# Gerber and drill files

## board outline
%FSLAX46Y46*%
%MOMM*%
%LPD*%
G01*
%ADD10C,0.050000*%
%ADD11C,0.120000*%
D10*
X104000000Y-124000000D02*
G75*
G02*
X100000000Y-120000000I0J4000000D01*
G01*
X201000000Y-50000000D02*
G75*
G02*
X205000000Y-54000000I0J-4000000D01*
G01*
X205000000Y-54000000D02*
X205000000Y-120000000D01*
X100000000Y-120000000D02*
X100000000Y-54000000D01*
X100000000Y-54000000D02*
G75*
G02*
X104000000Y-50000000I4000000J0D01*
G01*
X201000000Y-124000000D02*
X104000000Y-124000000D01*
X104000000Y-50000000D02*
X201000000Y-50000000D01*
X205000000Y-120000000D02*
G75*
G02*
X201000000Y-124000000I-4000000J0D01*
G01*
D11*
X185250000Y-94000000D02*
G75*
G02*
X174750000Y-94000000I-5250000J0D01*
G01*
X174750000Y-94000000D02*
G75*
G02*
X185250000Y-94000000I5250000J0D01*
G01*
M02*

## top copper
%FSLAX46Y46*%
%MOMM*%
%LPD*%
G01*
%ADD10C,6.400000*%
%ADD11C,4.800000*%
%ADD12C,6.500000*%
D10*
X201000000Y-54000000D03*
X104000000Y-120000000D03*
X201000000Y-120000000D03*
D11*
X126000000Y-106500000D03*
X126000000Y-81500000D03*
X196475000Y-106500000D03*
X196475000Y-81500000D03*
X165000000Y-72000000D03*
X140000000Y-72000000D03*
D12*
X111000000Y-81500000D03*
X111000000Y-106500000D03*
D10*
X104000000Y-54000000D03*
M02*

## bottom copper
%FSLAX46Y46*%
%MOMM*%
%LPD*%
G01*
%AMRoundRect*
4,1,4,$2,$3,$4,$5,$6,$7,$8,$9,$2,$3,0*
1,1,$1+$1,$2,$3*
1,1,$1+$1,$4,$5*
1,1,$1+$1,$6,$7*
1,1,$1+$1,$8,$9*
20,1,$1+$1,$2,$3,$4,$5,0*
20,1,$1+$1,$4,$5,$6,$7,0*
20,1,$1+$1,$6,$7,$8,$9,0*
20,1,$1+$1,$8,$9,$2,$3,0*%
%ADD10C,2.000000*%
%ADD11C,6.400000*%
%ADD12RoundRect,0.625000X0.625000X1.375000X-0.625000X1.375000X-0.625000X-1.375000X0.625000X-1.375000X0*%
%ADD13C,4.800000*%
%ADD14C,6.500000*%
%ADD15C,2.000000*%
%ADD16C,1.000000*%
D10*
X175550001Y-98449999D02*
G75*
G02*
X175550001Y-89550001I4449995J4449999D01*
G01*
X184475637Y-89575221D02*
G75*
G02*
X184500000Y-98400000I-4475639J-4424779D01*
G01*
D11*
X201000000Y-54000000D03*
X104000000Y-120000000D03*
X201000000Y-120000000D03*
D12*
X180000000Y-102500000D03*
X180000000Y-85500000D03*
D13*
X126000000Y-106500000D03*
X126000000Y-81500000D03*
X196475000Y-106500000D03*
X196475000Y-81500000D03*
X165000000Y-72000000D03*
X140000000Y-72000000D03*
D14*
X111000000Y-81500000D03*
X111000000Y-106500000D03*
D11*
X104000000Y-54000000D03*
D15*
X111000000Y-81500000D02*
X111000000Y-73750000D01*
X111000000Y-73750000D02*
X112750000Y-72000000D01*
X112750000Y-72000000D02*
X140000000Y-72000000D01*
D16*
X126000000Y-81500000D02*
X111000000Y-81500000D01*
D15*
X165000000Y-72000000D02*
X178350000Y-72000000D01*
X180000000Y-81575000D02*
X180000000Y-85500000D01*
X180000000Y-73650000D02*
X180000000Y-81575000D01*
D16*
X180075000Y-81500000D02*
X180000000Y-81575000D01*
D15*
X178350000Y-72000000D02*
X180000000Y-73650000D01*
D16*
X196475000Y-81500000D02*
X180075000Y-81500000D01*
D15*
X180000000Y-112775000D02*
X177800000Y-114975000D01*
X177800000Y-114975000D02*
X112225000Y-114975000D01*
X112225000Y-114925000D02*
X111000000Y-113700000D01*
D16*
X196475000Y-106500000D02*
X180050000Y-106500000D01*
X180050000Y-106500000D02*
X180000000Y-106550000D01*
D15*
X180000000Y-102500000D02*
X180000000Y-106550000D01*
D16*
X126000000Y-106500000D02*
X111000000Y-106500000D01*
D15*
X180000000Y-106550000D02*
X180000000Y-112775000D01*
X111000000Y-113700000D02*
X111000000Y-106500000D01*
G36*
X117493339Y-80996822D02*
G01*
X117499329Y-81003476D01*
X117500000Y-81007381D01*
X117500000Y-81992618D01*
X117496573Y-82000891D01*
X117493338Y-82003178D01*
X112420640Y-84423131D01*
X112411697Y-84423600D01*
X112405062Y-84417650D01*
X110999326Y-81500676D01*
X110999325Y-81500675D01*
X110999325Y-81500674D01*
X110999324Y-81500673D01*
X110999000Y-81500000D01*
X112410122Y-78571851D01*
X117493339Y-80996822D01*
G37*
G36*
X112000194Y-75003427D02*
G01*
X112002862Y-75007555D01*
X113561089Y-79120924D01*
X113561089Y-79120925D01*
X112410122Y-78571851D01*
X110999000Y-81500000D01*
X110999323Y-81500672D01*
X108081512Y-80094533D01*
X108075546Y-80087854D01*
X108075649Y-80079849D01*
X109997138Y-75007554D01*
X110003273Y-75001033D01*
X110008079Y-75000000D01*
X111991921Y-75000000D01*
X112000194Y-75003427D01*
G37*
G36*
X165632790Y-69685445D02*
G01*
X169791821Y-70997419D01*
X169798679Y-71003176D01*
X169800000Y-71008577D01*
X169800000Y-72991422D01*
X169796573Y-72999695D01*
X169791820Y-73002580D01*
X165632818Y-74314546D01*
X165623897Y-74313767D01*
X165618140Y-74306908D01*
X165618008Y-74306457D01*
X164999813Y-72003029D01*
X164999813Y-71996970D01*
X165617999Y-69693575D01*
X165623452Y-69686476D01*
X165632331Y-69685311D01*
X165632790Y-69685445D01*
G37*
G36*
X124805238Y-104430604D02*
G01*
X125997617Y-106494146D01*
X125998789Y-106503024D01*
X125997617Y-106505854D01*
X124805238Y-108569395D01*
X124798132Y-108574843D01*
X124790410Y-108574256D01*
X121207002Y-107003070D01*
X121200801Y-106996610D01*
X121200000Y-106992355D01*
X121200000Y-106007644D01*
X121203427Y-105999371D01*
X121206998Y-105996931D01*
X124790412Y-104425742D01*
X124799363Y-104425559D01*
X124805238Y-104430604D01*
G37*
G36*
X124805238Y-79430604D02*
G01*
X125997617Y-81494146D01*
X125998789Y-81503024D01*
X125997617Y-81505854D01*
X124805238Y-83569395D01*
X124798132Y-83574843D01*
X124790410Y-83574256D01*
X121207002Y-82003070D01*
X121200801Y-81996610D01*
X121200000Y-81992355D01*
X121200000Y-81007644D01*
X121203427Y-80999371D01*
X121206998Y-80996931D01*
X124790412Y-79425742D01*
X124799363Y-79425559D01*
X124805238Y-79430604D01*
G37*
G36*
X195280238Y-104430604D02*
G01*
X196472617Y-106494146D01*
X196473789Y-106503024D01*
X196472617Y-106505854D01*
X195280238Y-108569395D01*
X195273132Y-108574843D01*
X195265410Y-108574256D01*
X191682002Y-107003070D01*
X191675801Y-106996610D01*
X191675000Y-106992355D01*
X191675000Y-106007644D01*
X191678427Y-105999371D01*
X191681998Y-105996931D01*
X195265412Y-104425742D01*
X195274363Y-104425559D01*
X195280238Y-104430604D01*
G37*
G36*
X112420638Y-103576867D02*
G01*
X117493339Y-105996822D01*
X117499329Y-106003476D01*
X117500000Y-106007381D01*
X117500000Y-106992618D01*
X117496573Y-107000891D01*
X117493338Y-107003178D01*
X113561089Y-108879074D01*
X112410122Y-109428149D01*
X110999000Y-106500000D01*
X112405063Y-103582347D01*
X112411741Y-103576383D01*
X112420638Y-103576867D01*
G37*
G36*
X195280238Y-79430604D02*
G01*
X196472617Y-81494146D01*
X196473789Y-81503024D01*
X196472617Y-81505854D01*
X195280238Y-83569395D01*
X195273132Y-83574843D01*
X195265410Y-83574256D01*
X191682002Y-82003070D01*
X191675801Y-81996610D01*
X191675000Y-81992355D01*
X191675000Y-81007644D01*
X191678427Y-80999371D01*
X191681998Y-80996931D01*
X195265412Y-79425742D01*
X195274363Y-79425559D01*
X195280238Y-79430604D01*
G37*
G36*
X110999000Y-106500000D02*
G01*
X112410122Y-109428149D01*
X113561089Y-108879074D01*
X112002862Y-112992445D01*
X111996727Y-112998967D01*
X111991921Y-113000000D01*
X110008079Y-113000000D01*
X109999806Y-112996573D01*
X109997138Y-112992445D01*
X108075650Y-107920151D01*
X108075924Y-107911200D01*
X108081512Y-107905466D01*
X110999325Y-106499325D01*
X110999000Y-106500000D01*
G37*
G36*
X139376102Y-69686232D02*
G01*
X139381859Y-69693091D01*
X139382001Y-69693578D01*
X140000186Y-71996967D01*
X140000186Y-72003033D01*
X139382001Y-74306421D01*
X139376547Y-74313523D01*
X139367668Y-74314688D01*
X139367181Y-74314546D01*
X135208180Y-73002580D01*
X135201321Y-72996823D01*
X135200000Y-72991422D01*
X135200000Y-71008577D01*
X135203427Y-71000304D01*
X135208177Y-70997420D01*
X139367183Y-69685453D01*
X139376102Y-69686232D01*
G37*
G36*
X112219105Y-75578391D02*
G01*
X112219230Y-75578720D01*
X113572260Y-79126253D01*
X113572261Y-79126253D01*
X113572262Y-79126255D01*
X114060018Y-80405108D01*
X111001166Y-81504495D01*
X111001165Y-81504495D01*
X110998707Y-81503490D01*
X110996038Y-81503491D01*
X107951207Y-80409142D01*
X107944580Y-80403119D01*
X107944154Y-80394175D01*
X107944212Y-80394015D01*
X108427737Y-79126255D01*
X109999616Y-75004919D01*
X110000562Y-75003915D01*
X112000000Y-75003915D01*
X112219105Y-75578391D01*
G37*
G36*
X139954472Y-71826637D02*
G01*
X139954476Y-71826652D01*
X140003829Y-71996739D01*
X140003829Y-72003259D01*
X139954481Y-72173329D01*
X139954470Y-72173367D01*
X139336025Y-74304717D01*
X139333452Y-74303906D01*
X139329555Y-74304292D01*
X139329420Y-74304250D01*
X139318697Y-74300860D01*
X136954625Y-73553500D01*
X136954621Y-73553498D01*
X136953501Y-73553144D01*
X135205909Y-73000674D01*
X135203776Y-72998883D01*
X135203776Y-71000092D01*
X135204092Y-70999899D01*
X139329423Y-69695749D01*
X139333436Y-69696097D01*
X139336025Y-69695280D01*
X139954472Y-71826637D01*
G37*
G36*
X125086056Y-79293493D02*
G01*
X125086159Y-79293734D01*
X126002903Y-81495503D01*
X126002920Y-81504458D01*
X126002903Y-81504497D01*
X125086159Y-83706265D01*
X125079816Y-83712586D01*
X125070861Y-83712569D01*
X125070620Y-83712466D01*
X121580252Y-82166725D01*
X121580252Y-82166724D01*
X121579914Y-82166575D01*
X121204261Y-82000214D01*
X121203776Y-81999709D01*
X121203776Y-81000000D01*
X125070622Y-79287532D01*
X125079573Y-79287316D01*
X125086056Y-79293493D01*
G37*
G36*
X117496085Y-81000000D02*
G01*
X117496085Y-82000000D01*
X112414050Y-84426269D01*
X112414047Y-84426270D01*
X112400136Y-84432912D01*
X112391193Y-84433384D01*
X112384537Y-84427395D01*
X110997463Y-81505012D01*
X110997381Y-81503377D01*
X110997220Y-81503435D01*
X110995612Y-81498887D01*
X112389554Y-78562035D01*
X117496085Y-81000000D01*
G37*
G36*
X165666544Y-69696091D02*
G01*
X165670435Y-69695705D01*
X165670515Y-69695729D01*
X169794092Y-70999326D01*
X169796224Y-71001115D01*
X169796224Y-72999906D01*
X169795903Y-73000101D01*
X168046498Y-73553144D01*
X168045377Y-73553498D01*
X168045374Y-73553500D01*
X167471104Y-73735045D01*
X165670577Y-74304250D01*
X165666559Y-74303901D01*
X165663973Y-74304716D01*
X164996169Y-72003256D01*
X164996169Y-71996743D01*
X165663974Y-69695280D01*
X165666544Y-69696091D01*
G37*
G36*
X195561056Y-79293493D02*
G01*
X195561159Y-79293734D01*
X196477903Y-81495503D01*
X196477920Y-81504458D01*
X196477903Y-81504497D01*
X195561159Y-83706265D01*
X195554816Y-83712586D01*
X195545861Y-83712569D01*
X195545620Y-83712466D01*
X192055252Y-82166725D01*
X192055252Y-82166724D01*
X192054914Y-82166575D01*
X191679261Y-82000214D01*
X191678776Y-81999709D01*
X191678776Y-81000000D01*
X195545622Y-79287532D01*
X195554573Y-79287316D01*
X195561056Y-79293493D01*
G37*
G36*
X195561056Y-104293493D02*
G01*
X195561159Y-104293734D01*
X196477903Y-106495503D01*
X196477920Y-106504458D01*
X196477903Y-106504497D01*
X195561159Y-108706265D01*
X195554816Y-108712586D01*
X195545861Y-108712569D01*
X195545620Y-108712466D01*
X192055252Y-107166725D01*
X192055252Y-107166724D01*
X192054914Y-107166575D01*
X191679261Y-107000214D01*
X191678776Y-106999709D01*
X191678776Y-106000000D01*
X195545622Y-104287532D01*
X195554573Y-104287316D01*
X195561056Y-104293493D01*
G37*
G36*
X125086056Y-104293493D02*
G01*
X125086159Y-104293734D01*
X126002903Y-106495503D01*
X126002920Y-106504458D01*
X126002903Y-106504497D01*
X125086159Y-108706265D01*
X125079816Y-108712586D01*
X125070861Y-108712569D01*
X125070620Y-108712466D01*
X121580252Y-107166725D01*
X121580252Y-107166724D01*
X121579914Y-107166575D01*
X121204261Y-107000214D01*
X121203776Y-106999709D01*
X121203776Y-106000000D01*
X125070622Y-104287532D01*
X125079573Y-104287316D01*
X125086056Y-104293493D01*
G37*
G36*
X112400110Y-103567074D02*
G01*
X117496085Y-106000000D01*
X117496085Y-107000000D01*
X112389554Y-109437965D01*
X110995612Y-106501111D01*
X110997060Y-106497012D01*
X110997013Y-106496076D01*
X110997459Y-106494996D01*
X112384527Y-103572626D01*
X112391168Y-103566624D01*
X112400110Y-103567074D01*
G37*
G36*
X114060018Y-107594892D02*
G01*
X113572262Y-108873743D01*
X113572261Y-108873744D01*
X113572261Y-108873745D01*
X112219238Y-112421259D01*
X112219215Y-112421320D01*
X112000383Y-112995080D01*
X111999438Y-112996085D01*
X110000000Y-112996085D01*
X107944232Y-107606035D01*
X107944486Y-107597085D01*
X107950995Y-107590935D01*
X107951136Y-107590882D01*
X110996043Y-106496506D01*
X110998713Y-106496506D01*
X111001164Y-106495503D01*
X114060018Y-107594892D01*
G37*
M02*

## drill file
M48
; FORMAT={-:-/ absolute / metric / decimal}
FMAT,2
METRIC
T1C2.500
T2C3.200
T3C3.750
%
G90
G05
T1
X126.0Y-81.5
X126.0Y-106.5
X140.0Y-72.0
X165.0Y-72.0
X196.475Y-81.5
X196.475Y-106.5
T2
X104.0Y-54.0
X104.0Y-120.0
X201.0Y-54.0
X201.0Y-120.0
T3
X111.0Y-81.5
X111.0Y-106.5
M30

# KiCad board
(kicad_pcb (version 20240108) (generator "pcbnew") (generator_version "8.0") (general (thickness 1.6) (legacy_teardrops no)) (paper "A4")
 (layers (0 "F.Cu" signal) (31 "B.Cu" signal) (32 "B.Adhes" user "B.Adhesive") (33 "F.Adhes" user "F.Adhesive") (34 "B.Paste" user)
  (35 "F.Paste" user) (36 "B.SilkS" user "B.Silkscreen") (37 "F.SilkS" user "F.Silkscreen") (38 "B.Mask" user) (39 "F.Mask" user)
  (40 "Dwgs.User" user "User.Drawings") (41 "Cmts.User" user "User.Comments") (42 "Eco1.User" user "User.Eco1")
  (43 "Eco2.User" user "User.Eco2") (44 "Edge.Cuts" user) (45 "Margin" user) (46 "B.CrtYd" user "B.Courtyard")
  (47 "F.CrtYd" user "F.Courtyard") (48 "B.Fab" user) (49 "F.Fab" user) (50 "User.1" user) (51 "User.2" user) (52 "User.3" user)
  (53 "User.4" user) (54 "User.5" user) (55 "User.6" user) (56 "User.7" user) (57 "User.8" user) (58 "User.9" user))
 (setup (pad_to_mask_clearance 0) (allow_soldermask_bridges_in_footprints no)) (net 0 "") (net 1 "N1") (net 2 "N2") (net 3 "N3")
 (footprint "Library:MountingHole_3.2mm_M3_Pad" (layer "F.Cu") (at 201 54)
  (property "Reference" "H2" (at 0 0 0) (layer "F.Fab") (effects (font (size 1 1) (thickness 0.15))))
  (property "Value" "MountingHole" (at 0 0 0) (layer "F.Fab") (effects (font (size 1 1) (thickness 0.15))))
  (pad "1" thru_hole circle (at 0 0) (size 6.4 6.4) (drill 3.2) (layers "*.Cu" "*.Mask") (remove_unused_layers no)
   (teardrops (best_length_ratio 0.5) (max_length 8) (best_width_ratio 1) (max_width 8) (curve_points 0) (filter_ratio 0.9) (enabled yes)
    (allow_two_segments yes) (prefer_zone_connections yes))))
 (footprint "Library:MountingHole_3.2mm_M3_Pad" (layer "F.Cu") (at 104 120)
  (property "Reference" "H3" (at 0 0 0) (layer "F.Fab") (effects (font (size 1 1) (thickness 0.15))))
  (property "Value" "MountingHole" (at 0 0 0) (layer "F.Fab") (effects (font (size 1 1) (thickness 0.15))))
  (pad "1" thru_hole circle (at 0 0) (size 6.4 6.4) (drill 3.2) (layers "*.Cu" "*.Mask") (remove_unused_layers no)
   (teardrops (best_length_ratio 0.5) (max_length 8) (best_width_ratio 1) (max_width 8) (curve_points 0) (filter_ratio 0.9) (enabled yes)
    (allow_two_segments yes) (prefer_zone_connections yes))))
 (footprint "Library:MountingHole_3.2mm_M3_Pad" (layer "F.Cu") (at 201 120)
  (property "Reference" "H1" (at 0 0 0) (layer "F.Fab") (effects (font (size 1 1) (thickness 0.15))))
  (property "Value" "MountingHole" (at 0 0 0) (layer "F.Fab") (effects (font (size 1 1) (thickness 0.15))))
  (pad "1" thru_hole circle (at 0 0) (size 6.4 6.4) (drill 3.2) (layers "*.Cu" "*.Mask") (remove_unused_layers no)
   (teardrops (best_length_ratio 0.5) (max_length 8) (best_width_ratio 1) (max_width 8) (curve_points 0) (filter_ratio 0.9) (enabled yes)
    (allow_two_segments yes) (prefer_zone_connections yes))))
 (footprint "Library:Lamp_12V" (layer "F.Cu") (at 180 94)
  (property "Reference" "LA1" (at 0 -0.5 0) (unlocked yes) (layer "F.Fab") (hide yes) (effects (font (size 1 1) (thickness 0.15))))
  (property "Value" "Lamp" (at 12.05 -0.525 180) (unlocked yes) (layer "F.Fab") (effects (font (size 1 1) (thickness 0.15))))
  (fp_arc (start -4.449999 4.449999) (mid -6.29325 0) (end -4.449999 -4.449999) (stroke (width 2) (type default)) (layer "B.Cu"))
  (fp_arc (start 4.475637 -4.424779) (mid 6.293623 -0.017375) (end 4.5 4.4) (stroke (width 2) (type default)) (layer "B.Cu"))
  (fp_circle (center 0 0) (end 5.25 0) (stroke (width 0.12) (type default)) (fill none) (layer "Edge.Cuts"))
  (pad "1" smd roundrect (at 0 8.5 180) (size 2.5 4) (layers "B.Cu" "B.Paste" "B.Mask") (roundrect_rratio 0.25) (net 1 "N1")
   (thermal_bridge_angle 45)
   (teardrops (best_length_ratio 0.5) (max_length 8) (best_width_ratio 1) (max_width 8) (curve_points 0) (filter_ratio 0.9) (enabled no)
    (allow_two_segments yes) (prefer_zone_connections yes)))
  (pad "2" smd roundrect (at 0 -8.5 180) (size 2.5 4) (layers "B.Cu" "B.Paste" "B.Mask") (roundrect_rratio 0.25) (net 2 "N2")
   (thermal_bridge_angle 45)
   (teardrops (best_length_ratio 0.5) (max_length 8) (best_width_ratio 1) (max_width 8) (curve_points 0) (filter_ratio 0.9) (enabled no)
    (allow_two_segments yes) (prefer_zone_connections yes))))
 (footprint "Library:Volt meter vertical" (layer "F.Cu") (at 126 94)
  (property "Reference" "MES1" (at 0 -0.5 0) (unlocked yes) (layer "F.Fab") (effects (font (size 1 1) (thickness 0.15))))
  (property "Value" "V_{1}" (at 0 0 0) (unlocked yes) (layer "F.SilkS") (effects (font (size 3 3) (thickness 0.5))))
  (pad "1" thru_hole circle (at 0 12.5 180) (size 4.8 4.8) (drill 2.5) (layers "*.Cu" "*.Mask") (remove_unused_layers no) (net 1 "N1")
   (teardrops (best_length_ratio 0.5) (max_length 8) (best_width_ratio 1) (max_width 8) (curve_points 0) (filter_ratio 0.9) (enabled yes)
    (allow_two_segments yes) (prefer_zone_connections yes)))
  (pad "2" thru_hole circle (at 0 -12.5 180) (size 4.8 4.8) (drill 2.5) (layers "*.Cu" "*.Mask") (remove_unused_layers no) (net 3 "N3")
   (teardrops (best_length_ratio 0.5) (max_length 8) (best_width_ratio 1) (max_width 8) (curve_points 0) (filter_ratio 0.9) (enabled yes)
    (allow_two_segments yes) (prefer_zone_connections yes))))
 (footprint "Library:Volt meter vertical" (layer "F.Cu") (at 196.475 94)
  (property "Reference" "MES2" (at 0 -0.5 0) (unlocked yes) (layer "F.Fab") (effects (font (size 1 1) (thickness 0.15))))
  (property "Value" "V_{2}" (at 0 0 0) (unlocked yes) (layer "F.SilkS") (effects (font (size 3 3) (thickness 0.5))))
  (pad "1" thru_hole circle (at 0 12.5 180) (size 4.8 4.8) (drill 2.5) (layers "*.Cu" "*.Mask") (remove_unused_layers no) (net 1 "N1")
   (teardrops (best_length_ratio 0.5) (max_length 8) (best_width_ratio 1) (max_width 8) (curve_points 0) (filter_ratio 0.9) (enabled yes)
    (allow_two_segments yes) (prefer_zone_connections yes)))
  (pad "2" thru_hole circle (at 0 -12.5 180) (size 4.8 4.8) (drill 2.5) (layers "*.Cu" "*.Mask") (remove_unused_layers no) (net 2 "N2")
   (teardrops (best_length_ratio 0.5) (max_length 8) (best_width_ratio 1) (max_width 8) (curve_points 0) (filter_ratio 0.9) (enabled yes)
    (allow_two_segments yes) (prefer_zone_connections yes))))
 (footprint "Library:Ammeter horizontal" (layer "F.Cu") (at 152.5 72)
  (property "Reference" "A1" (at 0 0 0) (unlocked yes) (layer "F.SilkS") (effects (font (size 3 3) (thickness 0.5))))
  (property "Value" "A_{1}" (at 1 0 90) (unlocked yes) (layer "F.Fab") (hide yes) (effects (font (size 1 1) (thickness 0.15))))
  (pad "1" thru_hole circle (at 12.5 0 270) (size 4.8 4.8) (drill 2.5) (layers "*.Cu" "*.Mask") (remove_unused_layers no) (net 2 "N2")
   (teardrops (best_length_ratio 0.5) (max_length 8) (best_width_ratio 1) (max_width 8) (curve_points 0) (filter_ratio 0.9) (enabled yes)
    (allow_two_segments yes) (prefer_zone_connections yes)))
  (pad "2" thru_hole circle (at -12.5 0 270) (size 4.8 4.8) (drill 2.5) (layers "*.Cu" "*.Mask") (remove_unused_layers no) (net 3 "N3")
   (teardrops (best_length_ratio 0.5) (max_length 8) (best_width_ratio 1) (max_width 8) (curve_points 0) (filter_ratio 0.9) (enabled yes)
    (allow_two_segments yes) (prefer_zone_connections yes))))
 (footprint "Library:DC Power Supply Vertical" (layer "F.Cu") (at 111 94)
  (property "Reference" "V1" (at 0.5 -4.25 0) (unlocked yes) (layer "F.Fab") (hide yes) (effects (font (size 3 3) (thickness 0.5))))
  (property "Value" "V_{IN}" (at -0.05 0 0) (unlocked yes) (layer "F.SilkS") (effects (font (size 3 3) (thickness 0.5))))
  (pad "1" thru_hole circle (at 0 -12.5) (size 6.5 6.5) (drill 3.75) (layers "*.Cu" "*.Mask") (remove_unused_layers no) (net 3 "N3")
   (teardrops (best_length_ratio 0.5) (max_length 8) (best_width_ratio 1) (max_width 8) (curve_points 0) (filter_ratio 0.9) (enabled yes)
    (allow_two_segments yes) (prefer_zone_connections yes)))
  (pad "2" thru_hole circle (at 0 12.5) (size 6.5 6.5) (drill 3.75) (layers "*.Cu" "*.Mask") (remove_unused_layers no) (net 1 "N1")
   (teardrops (best_length_ratio 0.5) (max_length 8) (best_width_ratio 1) (max_width 8) (curve_points 0) (filter_ratio 0.9) (enabled yes)
    (allow_two_segments yes) (prefer_zone_connections yes))))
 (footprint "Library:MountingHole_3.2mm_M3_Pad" (layer "F.Cu") (at 104 54)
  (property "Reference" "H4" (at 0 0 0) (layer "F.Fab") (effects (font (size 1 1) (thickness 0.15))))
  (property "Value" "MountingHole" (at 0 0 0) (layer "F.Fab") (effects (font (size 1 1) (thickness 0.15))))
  (pad "1" thru_hole circle (at 0 0) (size 6.4 6.4) (drill 3.2) (layers "*.Cu" "*.Mask") (remove_unused_layers no)
   (teardrops (best_length_ratio 0.5) (max_length 8) (best_width_ratio 1) (max_width 8) (curve_points 0) (filter_ratio 0.9) (enabled yes)
    (allow_two_segments yes) (prefer_zone_connections yes))))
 (gr_arc (start 104 124) (mid 101.171573 122.828427) (end 100 120) (stroke (width 0.05) (type default)) (layer "Edge.Cuts"))
 (gr_arc (start 201 50) (mid 203.828427 51.171573) (end 205 54) (stroke (width 0.05) (type default)) (layer "Edge.Cuts"))
 (gr_line (start 205 54) (end 205 120) (stroke (width 0.05) (type default)) (layer "Edge.Cuts"))
 (gr_line (start 100 120) (end 100 54) (stroke (width 0.05) (type default)) (layer "Edge.Cuts"))
 (gr_arc (start 100 54) (mid 101.171573 51.171573) (end 104 50) (stroke (width 0.05) (type default)) (layer "Edge.Cuts"))
 (gr_line (start 201 124) (end 104 124) (stroke (width 0.05) (type default)) (layer "Edge.Cuts"))
 (gr_line (start 104 50) (end 201 50) (stroke (width 0.05) (type default)) (layer "Edge.Cuts"))
 (gr_arc (start 205 120) (mid 203.828427 122.828427) (end 201 124) (stroke (width 0.05) (type default)) (layer "Edge.Cuts"))
 (segment (start 111 81.5) (end 111 73.75) (width 2) (layer "B.Cu") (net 3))
 (segment (start 111 73.75) (end 112.75 72) (width 2) (layer "B.Cu") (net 3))
 (segment (start 112.75 72) (end 140 72) (width 2) (layer "B.Cu") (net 3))
 (segment (start 126 81.5) (end 111 81.5) (width 1) (layer "B.Cu") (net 3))
 (segment (start 165 72) (end 178.35 72) (width 2) (layer "B.Cu") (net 2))
 (segment (start 180 81.575) (end 180 85.5) (width 2) (layer "B.Cu") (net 2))
 (segment (start 180 73.65) (end 180 81.575) (width 2) (layer "B.Cu") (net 2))
 (segment (start 180.075 81.5) (end 180 81.575) (width 1) (layer "B.Cu") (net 2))
 (segment (start 178.35 72) (end 180 73.65) (width 2) (layer "B.Cu") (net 2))
 (segment (start 196.475 81.5) (end 180.075 81.5) (width 1) (layer "B.Cu") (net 2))
 (segment (start 180 112.775) (end 177.8 114.975) (width 2) (layer "B.Cu") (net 1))
 (segment (start 177.8 114.975) (end 112.225 114.975) (width 2) (layer "B.Cu") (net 1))
 (segment (start 112.225 114.925) (end 111 113.7) (width 2) (layer "B.Cu") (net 1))
 (segment (start 196.475 106.5) (end 180.05 106.5) (width 1) (layer "B.Cu") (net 1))
 (segment (start 180.05 106.5) (end 180 106.55) (width 1) (layer "B.Cu") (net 1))
 (segment (start 180 102.5) (end 180 106.55) (width 2) (layer "B.Cu") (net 1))
 (segment (start 126 106.5) (end 111 106.5) (width 1) (layer "B.Cu") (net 1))
 (segment (start 180 106.55) (end 180 112.775) (width 2) (layer "B.Cu") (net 1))
 (segment (start 111 113.7) (end 111 106.5) (width 2) (layer "B.Cu") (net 1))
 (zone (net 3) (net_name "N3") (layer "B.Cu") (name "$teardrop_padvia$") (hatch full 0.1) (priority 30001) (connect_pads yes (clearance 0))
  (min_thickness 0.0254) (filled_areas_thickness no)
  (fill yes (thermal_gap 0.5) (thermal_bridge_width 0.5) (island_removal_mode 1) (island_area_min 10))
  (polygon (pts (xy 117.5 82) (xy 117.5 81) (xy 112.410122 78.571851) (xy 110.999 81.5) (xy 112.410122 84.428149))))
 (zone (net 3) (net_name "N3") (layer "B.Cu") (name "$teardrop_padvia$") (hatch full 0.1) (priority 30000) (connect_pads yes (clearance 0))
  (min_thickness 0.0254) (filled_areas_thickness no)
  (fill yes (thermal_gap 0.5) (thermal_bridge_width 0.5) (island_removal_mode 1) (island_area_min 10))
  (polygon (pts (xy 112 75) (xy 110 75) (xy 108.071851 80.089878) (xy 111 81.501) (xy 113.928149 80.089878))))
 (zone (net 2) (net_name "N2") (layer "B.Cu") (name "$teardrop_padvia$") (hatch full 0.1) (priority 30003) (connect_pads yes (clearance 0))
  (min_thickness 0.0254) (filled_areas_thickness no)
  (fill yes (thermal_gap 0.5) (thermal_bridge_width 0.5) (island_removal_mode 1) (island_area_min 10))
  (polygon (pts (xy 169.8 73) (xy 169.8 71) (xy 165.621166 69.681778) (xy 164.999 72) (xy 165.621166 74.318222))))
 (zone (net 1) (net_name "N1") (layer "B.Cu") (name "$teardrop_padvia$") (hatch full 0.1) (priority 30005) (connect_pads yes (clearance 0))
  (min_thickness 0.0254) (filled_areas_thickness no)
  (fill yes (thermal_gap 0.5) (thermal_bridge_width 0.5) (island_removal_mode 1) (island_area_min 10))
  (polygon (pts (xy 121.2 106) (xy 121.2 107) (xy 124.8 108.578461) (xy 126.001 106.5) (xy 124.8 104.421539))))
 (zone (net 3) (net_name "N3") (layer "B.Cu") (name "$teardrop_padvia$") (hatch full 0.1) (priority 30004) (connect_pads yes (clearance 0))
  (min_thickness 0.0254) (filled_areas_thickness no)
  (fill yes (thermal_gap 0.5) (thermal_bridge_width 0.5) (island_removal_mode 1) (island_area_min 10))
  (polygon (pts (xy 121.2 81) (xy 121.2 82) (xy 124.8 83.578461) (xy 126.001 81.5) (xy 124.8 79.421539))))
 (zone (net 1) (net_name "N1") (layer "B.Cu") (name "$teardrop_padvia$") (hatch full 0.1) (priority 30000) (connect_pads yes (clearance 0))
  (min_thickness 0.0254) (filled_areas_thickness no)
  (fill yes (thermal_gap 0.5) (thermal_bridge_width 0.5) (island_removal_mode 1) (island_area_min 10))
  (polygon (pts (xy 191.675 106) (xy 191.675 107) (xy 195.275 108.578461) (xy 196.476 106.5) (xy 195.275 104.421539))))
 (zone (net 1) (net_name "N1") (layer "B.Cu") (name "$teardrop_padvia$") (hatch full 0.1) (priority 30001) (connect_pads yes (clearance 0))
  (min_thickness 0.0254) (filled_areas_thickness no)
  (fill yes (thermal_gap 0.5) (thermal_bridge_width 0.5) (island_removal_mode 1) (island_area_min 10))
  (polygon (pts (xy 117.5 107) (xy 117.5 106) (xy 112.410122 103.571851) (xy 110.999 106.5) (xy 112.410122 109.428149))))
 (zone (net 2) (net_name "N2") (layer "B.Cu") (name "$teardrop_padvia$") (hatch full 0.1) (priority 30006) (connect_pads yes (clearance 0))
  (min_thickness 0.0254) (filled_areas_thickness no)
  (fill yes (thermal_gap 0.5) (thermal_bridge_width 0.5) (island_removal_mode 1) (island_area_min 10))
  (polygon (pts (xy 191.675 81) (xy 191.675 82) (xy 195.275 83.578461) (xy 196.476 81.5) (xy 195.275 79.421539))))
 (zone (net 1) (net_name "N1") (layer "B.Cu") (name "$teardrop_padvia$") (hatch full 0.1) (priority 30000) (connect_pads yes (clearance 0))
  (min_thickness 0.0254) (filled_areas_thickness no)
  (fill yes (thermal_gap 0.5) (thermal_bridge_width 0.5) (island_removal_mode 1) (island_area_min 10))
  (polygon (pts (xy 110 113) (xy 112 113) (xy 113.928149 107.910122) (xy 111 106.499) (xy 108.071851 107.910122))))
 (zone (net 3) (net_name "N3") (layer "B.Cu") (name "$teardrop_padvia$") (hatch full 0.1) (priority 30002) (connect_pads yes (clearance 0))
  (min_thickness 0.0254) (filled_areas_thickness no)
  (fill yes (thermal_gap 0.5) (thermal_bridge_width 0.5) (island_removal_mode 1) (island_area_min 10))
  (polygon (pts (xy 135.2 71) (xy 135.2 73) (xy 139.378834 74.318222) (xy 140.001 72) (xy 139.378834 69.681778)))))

